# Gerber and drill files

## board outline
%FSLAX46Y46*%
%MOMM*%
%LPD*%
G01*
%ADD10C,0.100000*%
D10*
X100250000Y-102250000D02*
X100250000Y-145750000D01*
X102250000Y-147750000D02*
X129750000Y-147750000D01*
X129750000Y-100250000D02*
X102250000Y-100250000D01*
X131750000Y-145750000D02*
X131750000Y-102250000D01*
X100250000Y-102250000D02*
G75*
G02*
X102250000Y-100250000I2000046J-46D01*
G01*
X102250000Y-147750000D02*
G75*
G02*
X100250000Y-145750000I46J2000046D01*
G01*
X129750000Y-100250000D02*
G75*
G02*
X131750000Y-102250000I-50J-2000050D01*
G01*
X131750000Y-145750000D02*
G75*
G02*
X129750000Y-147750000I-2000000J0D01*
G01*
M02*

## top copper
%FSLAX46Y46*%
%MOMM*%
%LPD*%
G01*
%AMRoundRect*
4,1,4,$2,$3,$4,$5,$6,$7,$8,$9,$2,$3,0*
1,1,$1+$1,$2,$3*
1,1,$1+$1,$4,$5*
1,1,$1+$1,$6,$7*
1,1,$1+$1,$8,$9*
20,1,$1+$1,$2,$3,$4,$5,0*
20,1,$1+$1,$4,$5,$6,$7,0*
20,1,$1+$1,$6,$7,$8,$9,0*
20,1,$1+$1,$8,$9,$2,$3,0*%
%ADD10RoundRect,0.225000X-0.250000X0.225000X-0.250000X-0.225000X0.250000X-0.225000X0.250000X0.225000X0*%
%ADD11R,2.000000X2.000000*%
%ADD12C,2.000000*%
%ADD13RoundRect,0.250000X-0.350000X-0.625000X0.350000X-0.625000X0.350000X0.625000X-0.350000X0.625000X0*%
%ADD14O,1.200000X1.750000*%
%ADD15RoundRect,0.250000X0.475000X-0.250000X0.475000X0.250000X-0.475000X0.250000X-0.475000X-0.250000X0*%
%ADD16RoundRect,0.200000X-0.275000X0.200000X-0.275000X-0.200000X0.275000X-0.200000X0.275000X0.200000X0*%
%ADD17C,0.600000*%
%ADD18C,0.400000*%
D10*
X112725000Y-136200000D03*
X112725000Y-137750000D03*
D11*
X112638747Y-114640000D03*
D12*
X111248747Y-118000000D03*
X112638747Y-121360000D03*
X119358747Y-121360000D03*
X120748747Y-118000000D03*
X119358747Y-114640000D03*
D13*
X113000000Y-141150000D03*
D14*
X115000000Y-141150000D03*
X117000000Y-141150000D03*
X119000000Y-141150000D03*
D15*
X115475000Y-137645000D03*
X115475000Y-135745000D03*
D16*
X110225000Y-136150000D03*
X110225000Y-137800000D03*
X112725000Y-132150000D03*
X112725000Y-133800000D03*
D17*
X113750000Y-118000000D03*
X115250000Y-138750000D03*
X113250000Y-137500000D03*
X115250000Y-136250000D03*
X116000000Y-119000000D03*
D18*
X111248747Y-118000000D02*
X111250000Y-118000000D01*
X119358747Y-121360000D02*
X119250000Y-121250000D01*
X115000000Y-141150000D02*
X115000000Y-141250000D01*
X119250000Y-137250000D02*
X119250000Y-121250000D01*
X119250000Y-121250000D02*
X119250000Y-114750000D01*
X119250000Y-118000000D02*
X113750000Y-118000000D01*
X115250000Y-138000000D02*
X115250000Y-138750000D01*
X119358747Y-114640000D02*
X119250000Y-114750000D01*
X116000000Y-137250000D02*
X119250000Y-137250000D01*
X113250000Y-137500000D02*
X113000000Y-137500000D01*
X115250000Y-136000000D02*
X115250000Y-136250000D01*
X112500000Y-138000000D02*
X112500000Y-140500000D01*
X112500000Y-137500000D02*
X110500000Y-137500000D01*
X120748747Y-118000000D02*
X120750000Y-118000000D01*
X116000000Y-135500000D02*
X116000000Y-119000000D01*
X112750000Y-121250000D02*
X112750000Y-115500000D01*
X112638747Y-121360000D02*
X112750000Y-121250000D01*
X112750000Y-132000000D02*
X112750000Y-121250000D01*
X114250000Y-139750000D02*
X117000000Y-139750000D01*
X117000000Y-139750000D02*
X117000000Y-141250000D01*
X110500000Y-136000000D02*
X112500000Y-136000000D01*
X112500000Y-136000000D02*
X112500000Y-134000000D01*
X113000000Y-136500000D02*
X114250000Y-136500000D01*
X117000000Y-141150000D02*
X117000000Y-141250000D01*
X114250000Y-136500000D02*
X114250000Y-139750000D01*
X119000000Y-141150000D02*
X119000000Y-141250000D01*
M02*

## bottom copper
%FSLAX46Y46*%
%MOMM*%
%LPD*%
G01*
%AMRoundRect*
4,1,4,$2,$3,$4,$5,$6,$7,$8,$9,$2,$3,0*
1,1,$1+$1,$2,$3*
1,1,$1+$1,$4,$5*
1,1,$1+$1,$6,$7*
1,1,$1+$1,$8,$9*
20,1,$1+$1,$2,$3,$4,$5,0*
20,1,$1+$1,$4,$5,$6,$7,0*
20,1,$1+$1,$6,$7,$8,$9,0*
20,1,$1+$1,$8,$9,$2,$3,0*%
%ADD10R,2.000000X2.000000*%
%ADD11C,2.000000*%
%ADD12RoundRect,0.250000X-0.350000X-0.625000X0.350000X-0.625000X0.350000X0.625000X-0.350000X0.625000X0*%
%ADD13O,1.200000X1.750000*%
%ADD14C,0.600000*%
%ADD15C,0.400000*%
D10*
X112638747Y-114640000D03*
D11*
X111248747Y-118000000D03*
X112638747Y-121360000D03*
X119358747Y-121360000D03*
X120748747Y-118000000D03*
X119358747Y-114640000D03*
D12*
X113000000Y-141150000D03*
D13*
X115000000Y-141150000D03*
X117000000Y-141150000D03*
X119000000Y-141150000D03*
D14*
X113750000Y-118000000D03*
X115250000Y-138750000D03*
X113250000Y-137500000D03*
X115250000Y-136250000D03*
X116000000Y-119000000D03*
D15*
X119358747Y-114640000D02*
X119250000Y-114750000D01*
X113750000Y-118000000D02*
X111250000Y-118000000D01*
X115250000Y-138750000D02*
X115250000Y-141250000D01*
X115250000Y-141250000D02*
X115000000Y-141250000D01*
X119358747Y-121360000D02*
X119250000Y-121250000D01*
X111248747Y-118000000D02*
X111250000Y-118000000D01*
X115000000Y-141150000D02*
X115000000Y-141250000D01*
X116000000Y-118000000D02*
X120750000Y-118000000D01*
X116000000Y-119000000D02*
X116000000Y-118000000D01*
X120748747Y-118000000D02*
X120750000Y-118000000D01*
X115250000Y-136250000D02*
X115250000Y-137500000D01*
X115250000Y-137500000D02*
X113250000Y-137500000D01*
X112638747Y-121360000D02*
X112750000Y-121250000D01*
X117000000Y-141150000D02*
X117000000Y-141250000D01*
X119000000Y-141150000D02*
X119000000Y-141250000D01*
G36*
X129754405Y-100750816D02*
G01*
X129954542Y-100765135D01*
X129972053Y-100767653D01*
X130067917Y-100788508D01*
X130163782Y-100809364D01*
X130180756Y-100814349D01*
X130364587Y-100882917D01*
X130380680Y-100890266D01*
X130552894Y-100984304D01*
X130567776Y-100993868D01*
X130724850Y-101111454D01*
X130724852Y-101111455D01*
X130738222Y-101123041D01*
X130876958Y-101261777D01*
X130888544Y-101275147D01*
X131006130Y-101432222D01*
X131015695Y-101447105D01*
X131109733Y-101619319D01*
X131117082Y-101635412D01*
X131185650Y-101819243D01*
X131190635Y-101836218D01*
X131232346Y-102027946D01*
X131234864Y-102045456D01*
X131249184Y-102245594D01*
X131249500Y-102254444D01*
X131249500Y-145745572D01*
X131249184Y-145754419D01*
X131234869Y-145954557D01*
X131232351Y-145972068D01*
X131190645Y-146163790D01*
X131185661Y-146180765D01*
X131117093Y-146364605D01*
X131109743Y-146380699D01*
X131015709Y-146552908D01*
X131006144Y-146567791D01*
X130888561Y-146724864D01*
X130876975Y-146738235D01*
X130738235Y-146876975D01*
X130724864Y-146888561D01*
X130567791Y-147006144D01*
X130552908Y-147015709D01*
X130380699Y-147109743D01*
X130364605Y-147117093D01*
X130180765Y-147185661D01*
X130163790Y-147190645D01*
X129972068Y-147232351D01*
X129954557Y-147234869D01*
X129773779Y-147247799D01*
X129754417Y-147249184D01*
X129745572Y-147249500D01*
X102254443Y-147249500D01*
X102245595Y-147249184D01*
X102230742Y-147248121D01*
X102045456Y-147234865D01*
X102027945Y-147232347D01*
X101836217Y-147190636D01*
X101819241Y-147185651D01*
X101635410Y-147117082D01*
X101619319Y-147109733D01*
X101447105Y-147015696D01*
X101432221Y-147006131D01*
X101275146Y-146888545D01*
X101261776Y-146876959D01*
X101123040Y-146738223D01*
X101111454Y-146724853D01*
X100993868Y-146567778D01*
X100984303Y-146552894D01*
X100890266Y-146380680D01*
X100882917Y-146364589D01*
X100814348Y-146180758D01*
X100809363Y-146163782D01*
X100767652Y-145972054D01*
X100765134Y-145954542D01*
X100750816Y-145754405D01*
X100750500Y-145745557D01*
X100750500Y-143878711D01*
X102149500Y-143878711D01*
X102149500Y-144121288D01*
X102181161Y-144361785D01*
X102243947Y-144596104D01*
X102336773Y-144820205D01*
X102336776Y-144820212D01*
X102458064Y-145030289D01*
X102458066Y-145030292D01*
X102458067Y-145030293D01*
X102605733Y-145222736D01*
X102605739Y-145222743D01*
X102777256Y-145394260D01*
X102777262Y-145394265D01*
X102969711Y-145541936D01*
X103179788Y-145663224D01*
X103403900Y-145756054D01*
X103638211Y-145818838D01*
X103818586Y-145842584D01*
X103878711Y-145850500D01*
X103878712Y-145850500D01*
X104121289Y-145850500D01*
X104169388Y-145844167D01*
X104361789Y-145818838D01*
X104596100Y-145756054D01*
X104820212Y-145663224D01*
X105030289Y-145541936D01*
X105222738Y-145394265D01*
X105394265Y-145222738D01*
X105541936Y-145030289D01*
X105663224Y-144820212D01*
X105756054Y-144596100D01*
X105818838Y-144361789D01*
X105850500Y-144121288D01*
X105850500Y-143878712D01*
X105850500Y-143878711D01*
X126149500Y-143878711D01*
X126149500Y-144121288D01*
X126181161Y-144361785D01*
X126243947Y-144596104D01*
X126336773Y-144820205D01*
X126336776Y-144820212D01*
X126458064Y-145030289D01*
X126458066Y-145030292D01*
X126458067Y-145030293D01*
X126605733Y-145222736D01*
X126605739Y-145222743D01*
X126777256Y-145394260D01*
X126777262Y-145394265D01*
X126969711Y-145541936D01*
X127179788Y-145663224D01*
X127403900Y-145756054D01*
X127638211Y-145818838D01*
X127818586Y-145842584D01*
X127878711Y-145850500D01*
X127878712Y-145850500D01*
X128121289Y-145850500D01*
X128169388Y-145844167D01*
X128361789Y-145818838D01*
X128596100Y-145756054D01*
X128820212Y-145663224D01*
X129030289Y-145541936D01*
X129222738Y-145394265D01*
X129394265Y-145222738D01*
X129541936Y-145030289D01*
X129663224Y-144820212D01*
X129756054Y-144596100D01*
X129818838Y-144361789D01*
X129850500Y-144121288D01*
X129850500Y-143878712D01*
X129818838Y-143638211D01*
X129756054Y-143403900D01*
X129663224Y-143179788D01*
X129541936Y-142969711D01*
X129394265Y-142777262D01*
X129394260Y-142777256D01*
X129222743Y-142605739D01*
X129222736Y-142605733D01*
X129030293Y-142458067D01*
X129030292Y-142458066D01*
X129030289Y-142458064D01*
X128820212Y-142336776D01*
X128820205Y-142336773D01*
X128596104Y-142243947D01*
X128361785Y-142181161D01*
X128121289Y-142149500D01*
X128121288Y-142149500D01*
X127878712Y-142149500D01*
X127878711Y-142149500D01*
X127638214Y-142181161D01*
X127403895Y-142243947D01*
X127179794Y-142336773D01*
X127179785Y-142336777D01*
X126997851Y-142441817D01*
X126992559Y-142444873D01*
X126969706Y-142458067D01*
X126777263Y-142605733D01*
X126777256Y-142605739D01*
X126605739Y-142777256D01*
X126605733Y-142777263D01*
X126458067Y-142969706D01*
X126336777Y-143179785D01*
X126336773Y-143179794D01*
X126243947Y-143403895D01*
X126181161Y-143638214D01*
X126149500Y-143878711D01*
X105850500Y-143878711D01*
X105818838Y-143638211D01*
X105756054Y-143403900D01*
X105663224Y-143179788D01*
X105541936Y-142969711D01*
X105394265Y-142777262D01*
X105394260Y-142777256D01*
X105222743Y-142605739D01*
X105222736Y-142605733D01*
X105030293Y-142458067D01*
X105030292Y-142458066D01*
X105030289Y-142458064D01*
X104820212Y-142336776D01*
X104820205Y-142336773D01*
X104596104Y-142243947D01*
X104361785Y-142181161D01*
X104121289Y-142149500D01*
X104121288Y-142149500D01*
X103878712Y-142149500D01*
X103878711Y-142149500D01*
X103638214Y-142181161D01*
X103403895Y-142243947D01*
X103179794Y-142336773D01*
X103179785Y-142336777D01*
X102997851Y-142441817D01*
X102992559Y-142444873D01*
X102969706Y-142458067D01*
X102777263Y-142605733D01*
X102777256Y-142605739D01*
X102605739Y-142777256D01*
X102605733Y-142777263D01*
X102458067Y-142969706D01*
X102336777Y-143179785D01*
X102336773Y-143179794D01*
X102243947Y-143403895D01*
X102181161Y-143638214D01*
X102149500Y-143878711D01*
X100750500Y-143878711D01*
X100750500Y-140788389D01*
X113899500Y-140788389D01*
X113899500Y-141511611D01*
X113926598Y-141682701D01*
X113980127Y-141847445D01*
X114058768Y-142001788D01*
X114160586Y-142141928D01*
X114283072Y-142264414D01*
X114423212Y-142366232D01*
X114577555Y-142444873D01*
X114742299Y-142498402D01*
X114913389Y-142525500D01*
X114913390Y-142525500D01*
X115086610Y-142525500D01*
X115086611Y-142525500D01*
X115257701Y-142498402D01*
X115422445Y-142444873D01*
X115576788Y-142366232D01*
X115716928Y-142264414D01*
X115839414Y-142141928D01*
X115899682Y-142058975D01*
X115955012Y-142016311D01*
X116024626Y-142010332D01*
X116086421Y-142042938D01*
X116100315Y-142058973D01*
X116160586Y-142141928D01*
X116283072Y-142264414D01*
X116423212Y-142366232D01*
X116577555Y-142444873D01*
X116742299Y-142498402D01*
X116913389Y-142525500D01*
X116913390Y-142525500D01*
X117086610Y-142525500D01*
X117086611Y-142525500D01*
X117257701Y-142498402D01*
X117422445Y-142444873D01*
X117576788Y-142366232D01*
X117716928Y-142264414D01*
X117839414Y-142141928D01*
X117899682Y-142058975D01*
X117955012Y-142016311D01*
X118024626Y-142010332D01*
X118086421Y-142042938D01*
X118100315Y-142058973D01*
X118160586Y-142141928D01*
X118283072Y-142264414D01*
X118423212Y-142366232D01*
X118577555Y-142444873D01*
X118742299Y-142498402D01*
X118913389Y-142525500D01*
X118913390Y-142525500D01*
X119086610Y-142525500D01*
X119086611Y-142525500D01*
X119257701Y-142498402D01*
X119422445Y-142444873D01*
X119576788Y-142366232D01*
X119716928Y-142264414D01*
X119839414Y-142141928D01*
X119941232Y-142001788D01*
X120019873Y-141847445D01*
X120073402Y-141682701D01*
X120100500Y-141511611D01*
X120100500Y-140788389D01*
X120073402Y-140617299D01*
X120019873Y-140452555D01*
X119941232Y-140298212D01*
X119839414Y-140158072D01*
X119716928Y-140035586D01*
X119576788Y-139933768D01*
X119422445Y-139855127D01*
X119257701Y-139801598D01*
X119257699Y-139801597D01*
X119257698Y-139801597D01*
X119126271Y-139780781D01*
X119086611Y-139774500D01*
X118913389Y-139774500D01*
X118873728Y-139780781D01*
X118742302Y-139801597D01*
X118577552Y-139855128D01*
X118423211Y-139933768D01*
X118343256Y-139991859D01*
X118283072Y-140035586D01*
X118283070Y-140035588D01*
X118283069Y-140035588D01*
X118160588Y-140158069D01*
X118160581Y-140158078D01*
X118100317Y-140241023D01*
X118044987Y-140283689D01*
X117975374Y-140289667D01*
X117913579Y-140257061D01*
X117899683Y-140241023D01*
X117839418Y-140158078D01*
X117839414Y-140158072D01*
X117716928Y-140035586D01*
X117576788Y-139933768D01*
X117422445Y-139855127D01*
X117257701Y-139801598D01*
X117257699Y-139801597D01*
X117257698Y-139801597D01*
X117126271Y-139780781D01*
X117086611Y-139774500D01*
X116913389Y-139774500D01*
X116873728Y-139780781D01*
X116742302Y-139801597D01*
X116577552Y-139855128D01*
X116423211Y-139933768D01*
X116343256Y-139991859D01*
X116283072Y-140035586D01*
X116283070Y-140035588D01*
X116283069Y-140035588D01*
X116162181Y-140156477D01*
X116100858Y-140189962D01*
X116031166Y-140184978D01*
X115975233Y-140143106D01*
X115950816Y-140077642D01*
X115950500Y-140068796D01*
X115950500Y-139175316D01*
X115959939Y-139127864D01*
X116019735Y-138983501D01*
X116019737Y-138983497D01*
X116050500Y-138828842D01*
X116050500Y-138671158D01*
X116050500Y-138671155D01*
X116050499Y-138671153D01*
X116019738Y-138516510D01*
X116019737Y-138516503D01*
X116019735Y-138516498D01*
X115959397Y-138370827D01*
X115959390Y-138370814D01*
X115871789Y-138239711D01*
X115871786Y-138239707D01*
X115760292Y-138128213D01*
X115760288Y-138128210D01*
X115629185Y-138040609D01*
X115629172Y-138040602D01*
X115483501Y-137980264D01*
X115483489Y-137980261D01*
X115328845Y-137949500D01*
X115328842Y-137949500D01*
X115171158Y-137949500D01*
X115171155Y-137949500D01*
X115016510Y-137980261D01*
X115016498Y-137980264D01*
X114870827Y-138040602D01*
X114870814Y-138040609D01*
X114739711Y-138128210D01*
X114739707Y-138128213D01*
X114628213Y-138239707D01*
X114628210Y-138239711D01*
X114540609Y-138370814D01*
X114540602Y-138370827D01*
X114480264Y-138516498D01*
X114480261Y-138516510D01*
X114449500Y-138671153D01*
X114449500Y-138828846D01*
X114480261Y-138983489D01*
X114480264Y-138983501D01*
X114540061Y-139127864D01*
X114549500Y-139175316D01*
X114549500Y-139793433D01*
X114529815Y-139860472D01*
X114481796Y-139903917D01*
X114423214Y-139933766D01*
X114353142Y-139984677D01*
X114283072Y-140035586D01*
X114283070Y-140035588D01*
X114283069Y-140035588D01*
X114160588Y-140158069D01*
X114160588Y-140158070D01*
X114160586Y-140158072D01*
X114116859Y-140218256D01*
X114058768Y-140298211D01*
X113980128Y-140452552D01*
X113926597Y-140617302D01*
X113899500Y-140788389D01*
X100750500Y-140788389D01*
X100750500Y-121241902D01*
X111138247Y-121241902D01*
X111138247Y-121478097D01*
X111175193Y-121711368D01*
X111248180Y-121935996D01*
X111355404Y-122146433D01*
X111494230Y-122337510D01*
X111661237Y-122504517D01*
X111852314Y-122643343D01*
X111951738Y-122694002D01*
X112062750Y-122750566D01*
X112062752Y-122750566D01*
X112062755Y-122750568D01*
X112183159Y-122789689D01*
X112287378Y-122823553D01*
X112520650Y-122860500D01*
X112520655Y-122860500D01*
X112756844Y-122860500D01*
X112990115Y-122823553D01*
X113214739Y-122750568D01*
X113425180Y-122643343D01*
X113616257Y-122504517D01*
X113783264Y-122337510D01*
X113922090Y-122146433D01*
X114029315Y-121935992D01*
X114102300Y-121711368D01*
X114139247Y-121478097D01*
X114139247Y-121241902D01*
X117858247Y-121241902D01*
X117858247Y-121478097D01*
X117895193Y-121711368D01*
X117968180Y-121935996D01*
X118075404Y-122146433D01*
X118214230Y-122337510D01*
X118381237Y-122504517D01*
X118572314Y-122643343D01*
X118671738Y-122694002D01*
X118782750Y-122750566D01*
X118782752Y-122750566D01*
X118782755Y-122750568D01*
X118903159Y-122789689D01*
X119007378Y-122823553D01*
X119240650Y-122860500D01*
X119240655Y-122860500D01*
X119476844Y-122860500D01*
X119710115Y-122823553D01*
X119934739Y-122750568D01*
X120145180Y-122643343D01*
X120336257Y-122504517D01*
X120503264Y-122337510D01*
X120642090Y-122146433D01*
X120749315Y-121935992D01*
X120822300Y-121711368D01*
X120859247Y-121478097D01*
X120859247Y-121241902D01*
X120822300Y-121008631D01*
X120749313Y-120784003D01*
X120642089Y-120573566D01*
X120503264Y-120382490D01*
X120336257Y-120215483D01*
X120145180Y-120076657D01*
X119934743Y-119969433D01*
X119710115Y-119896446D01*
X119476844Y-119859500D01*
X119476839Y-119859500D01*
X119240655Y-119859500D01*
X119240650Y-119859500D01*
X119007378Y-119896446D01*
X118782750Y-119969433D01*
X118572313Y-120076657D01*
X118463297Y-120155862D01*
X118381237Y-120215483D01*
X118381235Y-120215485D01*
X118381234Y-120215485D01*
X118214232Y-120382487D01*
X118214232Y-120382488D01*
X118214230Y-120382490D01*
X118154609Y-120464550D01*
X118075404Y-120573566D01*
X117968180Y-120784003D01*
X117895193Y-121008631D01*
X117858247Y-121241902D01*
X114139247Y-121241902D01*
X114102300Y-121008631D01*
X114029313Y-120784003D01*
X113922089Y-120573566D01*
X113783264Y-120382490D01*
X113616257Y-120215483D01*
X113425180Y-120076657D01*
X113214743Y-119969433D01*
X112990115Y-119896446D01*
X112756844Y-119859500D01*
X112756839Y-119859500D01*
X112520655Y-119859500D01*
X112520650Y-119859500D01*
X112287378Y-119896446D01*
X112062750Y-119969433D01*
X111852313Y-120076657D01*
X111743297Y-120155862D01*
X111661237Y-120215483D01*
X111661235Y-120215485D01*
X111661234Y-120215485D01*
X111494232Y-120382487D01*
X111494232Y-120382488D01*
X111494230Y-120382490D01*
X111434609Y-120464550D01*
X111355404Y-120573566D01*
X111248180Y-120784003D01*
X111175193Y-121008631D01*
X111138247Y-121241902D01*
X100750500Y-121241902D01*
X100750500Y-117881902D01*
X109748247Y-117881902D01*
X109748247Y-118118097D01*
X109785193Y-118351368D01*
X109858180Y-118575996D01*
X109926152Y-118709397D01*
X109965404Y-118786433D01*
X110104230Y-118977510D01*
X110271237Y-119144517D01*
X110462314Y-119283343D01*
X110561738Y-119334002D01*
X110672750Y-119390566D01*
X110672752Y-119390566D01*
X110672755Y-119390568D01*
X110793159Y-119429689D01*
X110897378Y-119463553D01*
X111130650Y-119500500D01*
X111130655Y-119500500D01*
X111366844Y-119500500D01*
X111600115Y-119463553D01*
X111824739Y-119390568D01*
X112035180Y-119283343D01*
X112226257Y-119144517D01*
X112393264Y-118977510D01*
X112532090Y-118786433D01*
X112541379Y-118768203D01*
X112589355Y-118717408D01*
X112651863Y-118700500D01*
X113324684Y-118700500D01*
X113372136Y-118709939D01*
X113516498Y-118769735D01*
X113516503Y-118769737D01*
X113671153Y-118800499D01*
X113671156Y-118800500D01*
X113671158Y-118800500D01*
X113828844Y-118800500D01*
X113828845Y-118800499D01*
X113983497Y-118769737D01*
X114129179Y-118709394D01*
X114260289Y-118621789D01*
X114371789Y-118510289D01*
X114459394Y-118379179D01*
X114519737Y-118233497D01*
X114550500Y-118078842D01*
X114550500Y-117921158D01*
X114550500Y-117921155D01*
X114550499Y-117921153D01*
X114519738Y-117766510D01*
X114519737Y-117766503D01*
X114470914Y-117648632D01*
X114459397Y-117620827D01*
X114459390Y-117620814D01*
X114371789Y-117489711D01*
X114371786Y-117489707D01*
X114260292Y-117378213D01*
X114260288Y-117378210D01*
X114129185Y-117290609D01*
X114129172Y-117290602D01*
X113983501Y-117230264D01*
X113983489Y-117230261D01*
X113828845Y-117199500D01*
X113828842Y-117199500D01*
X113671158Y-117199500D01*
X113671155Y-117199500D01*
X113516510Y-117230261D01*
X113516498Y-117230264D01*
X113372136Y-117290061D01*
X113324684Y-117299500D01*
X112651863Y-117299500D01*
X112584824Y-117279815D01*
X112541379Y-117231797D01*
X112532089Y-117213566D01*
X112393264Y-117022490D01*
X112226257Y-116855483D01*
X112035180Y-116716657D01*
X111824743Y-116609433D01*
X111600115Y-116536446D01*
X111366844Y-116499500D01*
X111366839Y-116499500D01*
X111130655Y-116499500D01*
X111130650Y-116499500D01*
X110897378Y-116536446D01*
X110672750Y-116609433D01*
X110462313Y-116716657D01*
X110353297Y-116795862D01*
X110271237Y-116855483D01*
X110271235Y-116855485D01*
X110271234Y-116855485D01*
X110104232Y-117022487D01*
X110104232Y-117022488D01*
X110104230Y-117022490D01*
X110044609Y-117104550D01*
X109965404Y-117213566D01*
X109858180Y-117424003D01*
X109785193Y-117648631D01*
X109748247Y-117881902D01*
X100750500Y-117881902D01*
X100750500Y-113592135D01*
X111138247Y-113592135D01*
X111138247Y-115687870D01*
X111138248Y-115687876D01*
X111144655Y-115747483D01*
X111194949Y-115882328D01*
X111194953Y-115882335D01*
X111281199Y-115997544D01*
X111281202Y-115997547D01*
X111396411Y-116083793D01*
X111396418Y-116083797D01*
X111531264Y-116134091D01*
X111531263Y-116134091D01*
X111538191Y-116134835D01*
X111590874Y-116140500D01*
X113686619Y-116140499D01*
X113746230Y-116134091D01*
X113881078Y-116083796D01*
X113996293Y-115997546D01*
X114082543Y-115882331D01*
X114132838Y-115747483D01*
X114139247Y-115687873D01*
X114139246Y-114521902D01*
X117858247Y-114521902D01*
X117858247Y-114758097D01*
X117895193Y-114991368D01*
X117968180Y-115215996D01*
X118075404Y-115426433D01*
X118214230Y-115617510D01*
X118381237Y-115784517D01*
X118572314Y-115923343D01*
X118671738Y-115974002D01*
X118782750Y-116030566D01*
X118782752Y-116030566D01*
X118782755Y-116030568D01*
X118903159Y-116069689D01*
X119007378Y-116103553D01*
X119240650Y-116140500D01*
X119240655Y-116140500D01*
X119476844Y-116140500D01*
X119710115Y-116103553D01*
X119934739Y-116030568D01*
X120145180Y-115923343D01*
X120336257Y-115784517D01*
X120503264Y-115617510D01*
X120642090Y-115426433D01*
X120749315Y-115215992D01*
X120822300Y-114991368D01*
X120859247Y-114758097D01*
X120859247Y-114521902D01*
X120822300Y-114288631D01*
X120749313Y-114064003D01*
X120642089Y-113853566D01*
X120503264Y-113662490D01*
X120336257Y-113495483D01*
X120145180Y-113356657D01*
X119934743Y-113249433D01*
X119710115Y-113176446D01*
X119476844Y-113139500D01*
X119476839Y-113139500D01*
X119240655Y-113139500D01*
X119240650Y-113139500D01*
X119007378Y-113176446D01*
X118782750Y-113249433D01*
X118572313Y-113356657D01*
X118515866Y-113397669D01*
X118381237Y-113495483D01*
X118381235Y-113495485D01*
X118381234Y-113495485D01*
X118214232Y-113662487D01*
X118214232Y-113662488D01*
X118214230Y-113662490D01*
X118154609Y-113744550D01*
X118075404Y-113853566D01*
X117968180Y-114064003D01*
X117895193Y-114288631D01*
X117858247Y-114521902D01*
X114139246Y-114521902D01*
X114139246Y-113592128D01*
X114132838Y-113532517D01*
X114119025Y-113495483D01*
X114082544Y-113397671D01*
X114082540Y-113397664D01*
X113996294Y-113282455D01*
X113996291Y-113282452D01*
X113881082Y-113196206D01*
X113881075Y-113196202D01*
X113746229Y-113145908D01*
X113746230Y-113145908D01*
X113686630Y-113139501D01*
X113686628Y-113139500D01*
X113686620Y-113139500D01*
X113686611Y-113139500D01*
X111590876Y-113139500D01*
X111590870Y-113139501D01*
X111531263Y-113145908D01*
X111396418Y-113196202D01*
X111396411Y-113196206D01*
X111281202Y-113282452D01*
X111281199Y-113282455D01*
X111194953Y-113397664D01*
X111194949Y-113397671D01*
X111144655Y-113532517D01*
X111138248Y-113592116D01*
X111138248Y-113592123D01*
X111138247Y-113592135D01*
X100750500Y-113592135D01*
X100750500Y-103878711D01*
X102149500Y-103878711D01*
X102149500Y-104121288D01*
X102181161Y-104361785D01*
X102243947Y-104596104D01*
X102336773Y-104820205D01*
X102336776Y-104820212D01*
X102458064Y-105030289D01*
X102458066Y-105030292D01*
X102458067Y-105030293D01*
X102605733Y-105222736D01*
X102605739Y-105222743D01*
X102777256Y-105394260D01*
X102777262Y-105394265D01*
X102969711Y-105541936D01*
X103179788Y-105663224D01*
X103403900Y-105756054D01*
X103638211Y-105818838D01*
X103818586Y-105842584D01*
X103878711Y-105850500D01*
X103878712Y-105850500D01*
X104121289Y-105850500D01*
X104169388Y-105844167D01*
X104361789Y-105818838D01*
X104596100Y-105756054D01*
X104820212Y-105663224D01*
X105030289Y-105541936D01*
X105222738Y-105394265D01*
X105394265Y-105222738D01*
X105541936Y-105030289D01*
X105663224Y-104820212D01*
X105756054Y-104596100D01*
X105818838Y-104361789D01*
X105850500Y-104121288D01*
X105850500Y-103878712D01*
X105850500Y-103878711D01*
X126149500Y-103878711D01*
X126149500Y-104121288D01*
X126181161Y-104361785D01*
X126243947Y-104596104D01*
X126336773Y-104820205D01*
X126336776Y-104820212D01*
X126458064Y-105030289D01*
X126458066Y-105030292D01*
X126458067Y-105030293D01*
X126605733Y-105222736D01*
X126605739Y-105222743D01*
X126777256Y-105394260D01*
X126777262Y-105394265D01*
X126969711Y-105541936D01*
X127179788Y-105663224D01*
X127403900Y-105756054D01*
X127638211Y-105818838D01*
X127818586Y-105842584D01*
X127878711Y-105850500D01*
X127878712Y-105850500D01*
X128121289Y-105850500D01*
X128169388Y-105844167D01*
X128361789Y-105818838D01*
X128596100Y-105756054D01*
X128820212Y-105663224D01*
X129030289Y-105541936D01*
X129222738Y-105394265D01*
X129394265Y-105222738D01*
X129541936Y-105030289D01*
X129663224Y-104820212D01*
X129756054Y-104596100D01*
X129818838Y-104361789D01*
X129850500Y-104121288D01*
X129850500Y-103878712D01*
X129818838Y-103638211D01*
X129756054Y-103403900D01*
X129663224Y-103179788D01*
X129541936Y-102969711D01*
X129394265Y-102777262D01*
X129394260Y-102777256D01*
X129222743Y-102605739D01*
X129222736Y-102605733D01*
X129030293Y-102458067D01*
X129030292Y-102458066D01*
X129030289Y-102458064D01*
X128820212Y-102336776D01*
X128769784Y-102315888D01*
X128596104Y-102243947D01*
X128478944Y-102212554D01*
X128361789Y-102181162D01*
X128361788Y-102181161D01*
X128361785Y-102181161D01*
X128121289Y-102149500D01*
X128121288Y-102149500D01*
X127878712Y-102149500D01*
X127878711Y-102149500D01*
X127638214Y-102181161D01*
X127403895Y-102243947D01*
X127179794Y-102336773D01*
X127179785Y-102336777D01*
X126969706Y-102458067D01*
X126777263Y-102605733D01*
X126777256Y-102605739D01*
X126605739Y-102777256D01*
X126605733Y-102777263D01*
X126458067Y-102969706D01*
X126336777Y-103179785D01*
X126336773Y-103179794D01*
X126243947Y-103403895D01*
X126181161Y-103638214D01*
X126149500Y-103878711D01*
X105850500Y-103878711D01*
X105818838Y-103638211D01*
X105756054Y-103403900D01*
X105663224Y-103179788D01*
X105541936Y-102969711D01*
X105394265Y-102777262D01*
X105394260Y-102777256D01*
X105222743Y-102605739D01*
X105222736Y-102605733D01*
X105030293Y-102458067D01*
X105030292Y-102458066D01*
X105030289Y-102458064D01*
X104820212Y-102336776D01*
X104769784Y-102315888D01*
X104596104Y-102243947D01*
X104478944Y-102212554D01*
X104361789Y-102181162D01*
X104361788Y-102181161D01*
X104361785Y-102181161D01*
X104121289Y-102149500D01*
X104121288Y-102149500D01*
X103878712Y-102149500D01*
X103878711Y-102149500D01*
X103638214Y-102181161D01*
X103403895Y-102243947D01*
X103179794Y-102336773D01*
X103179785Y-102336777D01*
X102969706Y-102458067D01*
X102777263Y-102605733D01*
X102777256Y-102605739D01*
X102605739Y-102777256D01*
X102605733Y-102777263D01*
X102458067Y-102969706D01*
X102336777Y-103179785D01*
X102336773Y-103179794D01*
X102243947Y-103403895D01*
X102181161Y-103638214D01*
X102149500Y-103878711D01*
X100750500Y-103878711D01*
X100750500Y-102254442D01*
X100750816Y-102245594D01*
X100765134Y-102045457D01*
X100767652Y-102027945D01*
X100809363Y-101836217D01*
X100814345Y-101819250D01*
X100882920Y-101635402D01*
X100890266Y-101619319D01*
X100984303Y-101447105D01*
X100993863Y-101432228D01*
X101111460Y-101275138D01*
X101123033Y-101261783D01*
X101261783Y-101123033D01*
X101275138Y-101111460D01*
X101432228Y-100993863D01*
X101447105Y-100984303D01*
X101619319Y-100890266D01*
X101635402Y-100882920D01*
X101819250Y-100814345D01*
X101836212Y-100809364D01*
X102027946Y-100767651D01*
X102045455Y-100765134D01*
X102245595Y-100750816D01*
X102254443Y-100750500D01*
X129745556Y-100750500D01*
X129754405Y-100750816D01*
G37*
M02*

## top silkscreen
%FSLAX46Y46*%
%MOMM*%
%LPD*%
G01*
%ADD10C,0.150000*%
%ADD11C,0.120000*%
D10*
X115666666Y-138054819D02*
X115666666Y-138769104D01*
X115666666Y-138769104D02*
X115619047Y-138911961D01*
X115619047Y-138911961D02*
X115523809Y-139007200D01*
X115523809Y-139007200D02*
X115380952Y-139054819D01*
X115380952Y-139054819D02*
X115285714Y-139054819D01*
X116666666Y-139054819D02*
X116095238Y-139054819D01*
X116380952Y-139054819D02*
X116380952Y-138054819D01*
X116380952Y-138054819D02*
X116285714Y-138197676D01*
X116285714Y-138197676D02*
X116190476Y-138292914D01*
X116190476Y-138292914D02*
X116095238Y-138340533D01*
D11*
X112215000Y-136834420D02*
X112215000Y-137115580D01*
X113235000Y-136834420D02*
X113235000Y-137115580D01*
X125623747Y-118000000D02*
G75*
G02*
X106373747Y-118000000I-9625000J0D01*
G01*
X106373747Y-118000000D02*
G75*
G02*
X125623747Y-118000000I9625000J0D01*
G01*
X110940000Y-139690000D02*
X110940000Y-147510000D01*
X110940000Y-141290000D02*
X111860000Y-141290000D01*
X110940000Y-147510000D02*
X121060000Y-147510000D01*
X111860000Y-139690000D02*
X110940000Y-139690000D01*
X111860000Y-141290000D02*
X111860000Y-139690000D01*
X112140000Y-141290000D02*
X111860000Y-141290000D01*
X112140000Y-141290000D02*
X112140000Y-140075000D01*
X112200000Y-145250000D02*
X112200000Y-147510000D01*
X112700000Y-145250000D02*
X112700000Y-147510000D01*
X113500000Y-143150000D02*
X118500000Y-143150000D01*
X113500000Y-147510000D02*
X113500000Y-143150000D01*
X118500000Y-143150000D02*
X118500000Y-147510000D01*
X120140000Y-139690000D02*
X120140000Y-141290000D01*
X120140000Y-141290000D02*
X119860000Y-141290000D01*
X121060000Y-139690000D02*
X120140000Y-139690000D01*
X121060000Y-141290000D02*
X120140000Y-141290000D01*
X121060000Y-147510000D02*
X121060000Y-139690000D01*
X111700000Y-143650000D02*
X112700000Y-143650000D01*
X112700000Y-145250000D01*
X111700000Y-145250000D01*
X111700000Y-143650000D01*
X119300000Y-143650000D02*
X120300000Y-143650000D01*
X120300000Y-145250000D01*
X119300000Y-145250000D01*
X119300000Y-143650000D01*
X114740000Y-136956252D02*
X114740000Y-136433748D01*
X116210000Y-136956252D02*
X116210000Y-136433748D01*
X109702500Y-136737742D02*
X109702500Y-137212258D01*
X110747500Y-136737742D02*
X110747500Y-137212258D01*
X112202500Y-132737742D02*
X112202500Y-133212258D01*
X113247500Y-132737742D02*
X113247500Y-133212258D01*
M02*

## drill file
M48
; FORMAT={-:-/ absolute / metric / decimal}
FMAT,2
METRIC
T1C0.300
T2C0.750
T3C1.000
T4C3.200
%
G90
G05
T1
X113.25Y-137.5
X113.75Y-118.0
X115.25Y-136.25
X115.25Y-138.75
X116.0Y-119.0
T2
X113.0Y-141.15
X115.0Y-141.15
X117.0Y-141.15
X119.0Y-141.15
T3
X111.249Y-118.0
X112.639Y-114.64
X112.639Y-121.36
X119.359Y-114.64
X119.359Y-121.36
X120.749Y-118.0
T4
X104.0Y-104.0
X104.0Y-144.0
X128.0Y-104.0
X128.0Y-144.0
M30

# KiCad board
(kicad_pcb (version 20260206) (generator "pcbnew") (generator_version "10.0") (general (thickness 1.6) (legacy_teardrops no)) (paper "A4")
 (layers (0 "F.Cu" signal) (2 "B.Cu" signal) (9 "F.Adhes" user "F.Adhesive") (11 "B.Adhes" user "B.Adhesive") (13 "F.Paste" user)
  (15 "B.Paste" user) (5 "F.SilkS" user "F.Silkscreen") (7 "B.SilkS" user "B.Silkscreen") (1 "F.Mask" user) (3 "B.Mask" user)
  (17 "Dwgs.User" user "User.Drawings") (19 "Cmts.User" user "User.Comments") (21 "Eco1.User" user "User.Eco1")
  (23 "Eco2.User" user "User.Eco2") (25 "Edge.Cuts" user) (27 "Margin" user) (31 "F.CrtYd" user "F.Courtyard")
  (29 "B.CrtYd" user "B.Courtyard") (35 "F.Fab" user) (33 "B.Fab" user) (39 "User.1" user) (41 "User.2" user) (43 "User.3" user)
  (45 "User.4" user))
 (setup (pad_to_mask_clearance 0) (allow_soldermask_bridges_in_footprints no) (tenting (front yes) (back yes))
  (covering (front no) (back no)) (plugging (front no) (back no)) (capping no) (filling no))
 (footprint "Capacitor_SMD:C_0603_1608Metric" (layer "F.Cu") (at 112.725 136.975 -90)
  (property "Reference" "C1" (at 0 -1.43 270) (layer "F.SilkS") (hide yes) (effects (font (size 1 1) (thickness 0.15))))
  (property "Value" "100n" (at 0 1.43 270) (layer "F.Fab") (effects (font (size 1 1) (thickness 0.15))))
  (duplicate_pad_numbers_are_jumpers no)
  (fp_line (start -0.14058 0.51) (end 0.14058 0.51) (stroke (width 0.12) (type solid)) (layer "F.SilkS"))
  (fp_line (start -0.14058 -0.51) (end 0.14058 -0.51) (stroke (width 0.12) (type solid)) (layer "F.SilkS"))
  (pad "1" smd roundrect (at -0.775 0 270) (size 0.9 0.95) (layers "F.Cu" "F.Mask" "F.Paste") (roundrect_rratio 0.25) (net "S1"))
  (pad "2" smd roundrect (at 0.775 0 270) (size 0.9 0.95) (layers "F.Cu" "F.Mask" "F.Paste") (roundrect_rratio 0.25) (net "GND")))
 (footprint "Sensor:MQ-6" (layer "F.Cu") (at 112.638747 114.64)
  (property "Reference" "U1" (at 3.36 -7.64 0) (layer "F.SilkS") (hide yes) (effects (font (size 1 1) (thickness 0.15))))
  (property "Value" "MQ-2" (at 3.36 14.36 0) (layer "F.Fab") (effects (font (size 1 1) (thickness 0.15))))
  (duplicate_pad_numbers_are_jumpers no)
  (fp_circle (center 3.36 3.36) (end 12.985 3.36) (stroke (width 0.12) (type solid)) (fill no) (layer "F.SilkS"))
  (pad "1" thru_hole rect (at 0 0) (size 2 2) (drill 1) (layers "*.Cu" "*.Mask") (remove_unused_layers no) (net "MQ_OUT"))
  (pad "2" thru_hole circle (at -1.39 3.36) (size 2 2) (drill 1) (layers "*.Cu" "*.Mask") (remove_unused_layers no) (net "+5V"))
  (pad "3" thru_hole circle (at 0 6.72 90) (size 2 2) (drill 1) (layers "*.Cu" "*.Mask") (remove_unused_layers no) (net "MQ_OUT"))
  (pad "4" thru_hole circle (at 6.72 6.72 180) (size 2 2) (drill 1) (layers "*.Cu" "*.Mask") (remove_unused_layers no) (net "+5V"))
  (pad "5" thru_hole circle (at 8.11 3.36) (size 2 2) (drill 1) (layers "*.Cu" "*.Mask") (remove_unused_layers no) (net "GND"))
  (pad "6" thru_hole circle (at 6.72 0 270) (size 2 2) (drill 1) (layers "*.Cu" "*.Mask") (remove_unused_layers no) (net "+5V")))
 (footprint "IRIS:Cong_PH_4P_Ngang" (layer "F.Cu") (at 113 141.15)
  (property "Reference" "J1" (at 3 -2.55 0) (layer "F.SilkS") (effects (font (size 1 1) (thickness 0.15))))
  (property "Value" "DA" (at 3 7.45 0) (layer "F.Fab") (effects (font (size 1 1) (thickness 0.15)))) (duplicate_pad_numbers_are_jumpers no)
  (fp_line (start -2.06 -1.46) (end -2.06 6.36) (stroke (width 0.12) (type solid)) (layer "F.SilkS"))
  (fp_line (start -2.06 0.14) (end -1.14 0.14) (stroke (width 0.12) (type solid)) (layer "F.SilkS"))
  (fp_line (start -2.06 6.36) (end 8.06 6.36) (stroke (width 0.12) (type solid)) (layer "F.SilkS"))
  (fp_line (start -1.14 -1.46) (end -2.06 -1.46) (stroke (width 0.12) (type solid)) (layer "F.SilkS"))
  (fp_line (start -1.14 0.14) (end -1.14 -1.46) (stroke (width 0.12) (type solid)) (layer "F.SilkS"))
  (fp_line (start -0.86 0.14) (end -1.14 0.14) (stroke (width 0.12) (type solid)) (layer "F.SilkS"))
  (fp_line (start -0.86 0.14) (end -0.86 -1.075) (stroke (width 0.12) (type solid)) (layer "F.SilkS"))
  (fp_line (start -0.8 4.1) (end -0.8 6.36) (stroke (width 0.12) (type solid)) (layer "F.SilkS"))
  (fp_line (start -0.3 4.1) (end -0.3 6.36) (stroke (width 0.12) (type solid)) (layer "F.SilkS"))
  (fp_line (start 0.5 2) (end 5.5 2) (stroke (width 0.12) (type solid)) (layer "F.SilkS"))
  (fp_line (start 0.5 6.36) (end 0.5 2) (stroke (width 0.12) (type solid)) (layer "F.SilkS"))
  (fp_line (start 5.5 2) (end 5.5 6.36) (stroke (width 0.12) (type solid)) (layer "F.SilkS"))
  (fp_line (start 7.14 -1.46) (end 7.14 0.14) (stroke (width 0.12) (type solid)) (layer "F.SilkS"))
  (fp_line (start 7.14 0.14) (end 6.86 0.14) (stroke (width 0.12) (type solid)) (layer "F.SilkS"))
  (fp_line (start 8.06 -1.46) (end 7.14 -1.46) (stroke (width 0.12) (type solid)) (layer "F.SilkS"))
  (fp_line (start 8.06 0.14) (end 7.14 0.14) (stroke (width 0.12) (type solid)) (layer "F.SilkS"))
  (fp_line (start 8.06 6.36) (end 8.06 -1.46) (stroke (width 0.12) (type solid)) (layer "F.SilkS"))
  (fp_rect (start -1.3 2.5) (end -0.3 4.1) (stroke (width 0.12) (type solid)) (fill no) (layer "F.SilkS"))
  (fp_rect (start 6.3 2.5) (end 7.3 4.1) (stroke (width 0.12) (type solid)) (fill no) (layer "F.SilkS"))
  (pad "1" thru_hole roundrect (at 0 0) (size 1.2 1.75) (drill 0.75) (layers "*.Cu" "*.Mask") (remove_unused_layers no)
   (roundrect_rratio 0.208333) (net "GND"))
  (pad "2" thru_hole oval (at 2 0) (size 1.2 1.75) (drill 0.75) (layers "*.Cu" "*.Mask") (remove_unused_layers no) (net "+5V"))
  (pad "3" thru_hole oval (at 4 0) (size 1.2 1.75) (drill 0.75) (layers "*.Cu" "*.Mask") (remove_unused_layers no) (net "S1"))
  (pad "4" thru_hole oval (at 6 0) (size 1.2 1.75) (drill 0.75) (layers "*.Cu" "*.Mask") (remove_unused_layers no)
   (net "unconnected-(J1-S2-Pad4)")))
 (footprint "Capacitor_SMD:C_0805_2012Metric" (layer "F.Cu") (at 115.475 136.695 90)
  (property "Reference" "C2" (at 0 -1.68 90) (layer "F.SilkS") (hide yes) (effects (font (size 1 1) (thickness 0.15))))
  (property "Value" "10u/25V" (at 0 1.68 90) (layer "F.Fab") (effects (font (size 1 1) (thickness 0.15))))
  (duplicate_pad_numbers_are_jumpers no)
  (fp_line (start -0.261252 -0.735) (end 0.261252 -0.735) (stroke (width 0.12) (type solid)) (layer "F.SilkS"))
  (fp_line (start -0.261252 0.735) (end 0.261252 0.735) (stroke (width 0.12) (type solid)) (layer "F.SilkS"))
  (pad "1" smd roundrect (at -0.95 0 90) (size 1 1.45) (layers "F.Cu" "F.Mask" "F.Paste") (roundrect_rratio 0.25) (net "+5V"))
  (pad "2" smd roundrect (at 0.95 0 90) (size 1 1.45) (layers "F.Cu" "F.Mask" "F.Paste") (roundrect_rratio 0.25) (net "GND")))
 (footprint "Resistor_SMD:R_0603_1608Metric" (layer "F.Cu") (at 110.225 136.975 -90)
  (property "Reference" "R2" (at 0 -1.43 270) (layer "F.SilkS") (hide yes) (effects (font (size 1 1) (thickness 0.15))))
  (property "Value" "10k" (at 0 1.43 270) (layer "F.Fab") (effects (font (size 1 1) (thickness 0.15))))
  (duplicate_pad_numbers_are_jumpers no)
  (fp_line (start -0.237258 0.5225) (end 0.237258 0.5225) (stroke (width 0.12) (type solid)) (layer "F.SilkS"))
  (fp_line (start -0.237258 -0.5225) (end 0.237258 -0.5225) (stroke (width 0.12) (type solid)) (layer "F.SilkS"))
  (pad "1" smd roundrect (at -0.825 0 270) (size 0.8 0.95) (layers "F.Cu" "F.Mask" "F.Paste") (roundrect_rratio 0.25) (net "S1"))
  (pad "2" smd roundrect (at 0.825 0 270) (size 0.8 0.95) (layers "F.Cu" "F.Mask" "F.Paste") (roundrect_rratio 0.25) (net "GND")))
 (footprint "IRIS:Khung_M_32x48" (layer "F.Cu") (at 100 148)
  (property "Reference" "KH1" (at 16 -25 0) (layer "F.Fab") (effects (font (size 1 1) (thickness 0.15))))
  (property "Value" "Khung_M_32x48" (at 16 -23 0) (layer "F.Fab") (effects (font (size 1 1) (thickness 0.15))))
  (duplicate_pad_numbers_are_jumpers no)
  (fp_line (start 0.25 -45.75) (end 0.25 -2.25) (stroke (width 0.1) (type solid)) (layer "Edge.Cuts"))
  (fp_line (start 2.25 -0.25) (end 29.75 -0.25) (stroke (width 0.1) (type solid)) (layer "Edge.Cuts"))
  (fp_line (start 29.75 -47.75) (end 2.25 -47.75) (stroke (width 0.1) (type solid)) (layer "Edge.Cuts"))
  (fp_line (start 31.75 -2.25) (end 31.75 -45.75) (stroke (width 0.1) (type solid)) (layer "Edge.Cuts"))
  (fp_arc (start 0.25 -45.75) (mid 0.8358 -47.1642) (end 2.25 -47.75) (stroke (width 0.1) (type solid)) (layer "Edge.Cuts"))
  (fp_arc (start 2.25 -0.25) (mid 0.8358 -0.8358) (end 0.25 -2.25) (stroke (width 0.1) (type solid)) (layer "Edge.Cuts"))
  (fp_arc (start 29.75 -47.75) (mid 31.164199 -47.164199) (end 31.75 -45.75) (stroke (width 0.1) (type solid)) (layer "Edge.Cuts"))
  (fp_arc (start 31.75 -2.25) (mid 31.164214 -0.835786) (end 29.75 -0.25) (stroke (width 0.1) (type solid)) (layer "Edge.Cuts"))
  (pad "" np_thru_hole circle (at 4 -44) (size 3.2 3.2) (drill 3.2) (layers "*.Cu" "*.Mask"))
  (pad "" np_thru_hole circle (at 4 -4) (size 3.2 3.2) (drill 3.2) (layers "*.Cu" "*.Mask"))
  (pad "" np_thru_hole circle (at 28 -44) (size 3.2 3.2) (drill 3.2) (layers "*.Cu" "*.Mask"))
  (pad "" np_thru_hole circle (at 28 -4) (size 3.2 3.2) (drill 3.2) (layers "*.Cu" "*.Mask")))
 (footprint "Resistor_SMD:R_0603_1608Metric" (layer "F.Cu") (at 112.725 132.975 -90)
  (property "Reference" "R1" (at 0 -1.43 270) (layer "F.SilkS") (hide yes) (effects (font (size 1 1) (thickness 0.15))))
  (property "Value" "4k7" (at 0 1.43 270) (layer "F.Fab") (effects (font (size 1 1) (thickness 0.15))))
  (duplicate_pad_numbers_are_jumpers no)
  (fp_line (start -0.237258 0.5225) (end 0.237258 0.5225) (stroke (width 0.12) (type solid)) (layer "F.SilkS"))
  (fp_line (start -0.237258 -0.5225) (end 0.237258 -0.5225) (stroke (width 0.12) (type solid)) (layer "F.SilkS"))
  (pad "1" smd roundrect (at -0.825 0 270) (size 0.8 0.95) (layers "F.Cu" "F.Mask" "F.Paste") (roundrect_rratio 0.25) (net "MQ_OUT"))
  (pad "2" smd roundrect (at 0.825 0 270) (size 0.8 0.95) (layers "F.Cu" "F.Mask" "F.Paste") (roundrect_rratio 0.25) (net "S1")))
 (segment (start 111.248747 118) (end 111.25 118) (width 0.4) (layer "F.Cu") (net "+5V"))
 (segment (start 119.358747 121.36) (end 119.25 121.25) (width 0.4) (layer "F.Cu") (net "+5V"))
 (segment (start 115 141.15) (end 115 141.25) (width 0.4) (layer "F.Cu") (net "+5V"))
 (segment (start 119.25 137.25) (end 119.25 121.25) (width 0.4) (layer "F.Cu") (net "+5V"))
 (segment (start 119.25 121.25) (end 119.25 114.75) (width 0.4) (layer "F.Cu") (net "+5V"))
 (segment (start 119.25 118) (end 113.75 118) (width 0.4) (layer "F.Cu") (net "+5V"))
 (segment (start 115.25 138) (end 115.25 138.75) (width 0.4) (layer "F.Cu") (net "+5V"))
 (segment (start 119.358747 114.64) (end 119.25 114.75) (width 0.4) (layer "F.Cu") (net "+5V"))
 (segment (start 116 137.25) (end 119.25 137.25) (width 0.4) (layer "F.Cu") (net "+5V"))
 (via (at 113.75 118) (size 0.6) (drill 0.3) (layers "F.Cu" "B.Cu") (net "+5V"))
 (via (at 115.25 138.75) (size 0.6) (drill 0.3) (layers "F.Cu" "B.Cu") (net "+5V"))
 (segment (start 119.358747 114.64) (end 119.25 114.75) (width 0.4) (layer "B.Cu") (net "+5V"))
 (segment (start 113.75 118) (end 111.25 118) (width 0.4) (layer "B.Cu") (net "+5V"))
 (segment (start 115.25 138.75) (end 115.25 141.25) (width 0.4) (layer "B.Cu") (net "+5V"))
 (segment (start 115.25 141.25) (end 115 141.25) (width 0.4) (layer "B.Cu") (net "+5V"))
 (segment (start 119.358747 121.36) (end 119.25 121.25) (width 0.4) (layer "B.Cu") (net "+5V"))
 (segment (start 111.248747 118) (end 111.25 118) (width 0.4) (layer "B.Cu") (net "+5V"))
 (segment (start 115 141.15) (end 115 141.25) (width 0.4) (layer "B.Cu") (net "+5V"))
 (segment (start 113.25 137.5) (end 113 137.5) (width 0.4) (layer "F.Cu") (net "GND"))
 (segment (start 115.25 136) (end 115.25 136.25) (width 0.4) (layer "F.Cu") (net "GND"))
 (segment (start 112.5 138) (end 112.5 140.5) (width 0.4) (layer "F.Cu") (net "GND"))
 (segment (start 112.5 137.5) (end 110.5 137.5) (width 0.4) (layer "F.Cu") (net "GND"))
 (segment (start 120.748747 118) (end 120.75 118) (width 0.4) (layer "F.Cu") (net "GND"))
 (segment (start 116 135.5) (end 116 119) (width 0.4) (layer "F.Cu") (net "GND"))
 (via (at 113.25 137.5) (size 0.6) (drill 0.3) (layers "F.Cu" "B.Cu") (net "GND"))
 (via (at 115.25 136.25) (size 0.6) (drill 0.3) (layers "F.Cu" "B.Cu") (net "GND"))
 (via (at 116 119) (size 0.6) (drill 0.3) (layers "F.Cu" "B.Cu") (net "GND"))
 (segment (start 116 118) (end 120.75 118) (width 0.4) (layer "B.Cu") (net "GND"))
 (segment (start 116 119) (end 116 118) (width 0.4) (layer "B.Cu") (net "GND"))
 (segment (start 120.748747 118) (end 120.75 118) (width 0.4) (layer "B.Cu") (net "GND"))
 (segment (start 115.25 136.25) (end 115.25 137.5) (width 0.4) (layer "B.Cu") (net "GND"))
 (segment (start 115.25 137.5) (end 113.25 137.5) (width 0.4) (layer "B.Cu") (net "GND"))
 (segment (start 112.75 121.25) (end 112.75 115.5) (width 0.4) (layer "F.Cu") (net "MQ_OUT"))
 (segment (start 112.638747 121.36) (end 112.75 121.25) (width 0.4) (layer "F.Cu") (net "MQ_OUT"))
 (segment (start 112.75 132) (end 112.75 121.25) (width 0.4) (layer "F.Cu") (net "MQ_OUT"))
 (segment (start 112.638747 121.36) (end 112.75 121.25) (width 0.4) (layer "B.Cu") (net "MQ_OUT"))
 (segment (start 114.25 139.75) (end 117 139.75) (width 0.4) (layer "F.Cu") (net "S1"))
 (segment (start 117 139.75) (end 117 141.25) (width 0.4) (layer "F.Cu") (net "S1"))
 (segment (start 110.5 136) (end 112.5 136) (width 0.4) (layer "F.Cu") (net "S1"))
 (segment (start 112.5 136) (end 112.5 134) (width 0.4) (layer "F.Cu") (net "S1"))
 (segment (start 113 136.5) (end 114.25 136.5) (width 0.4) (layer "F.Cu") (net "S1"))
 (segment (start 117 141.15) (end 117 141.25) (width 0.4) (layer "F.Cu") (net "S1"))
 (segment (start 114.25 136.5) (end 114.25 139.75) (width 0.4) (layer "F.Cu") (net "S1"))
 (segment (start 117 141.15) (end 117 141.25) (width 0.4) (layer "B.Cu") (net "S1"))
 (segment (start 119 141.15) (end 119 141.25) (width 0.4) (layer "F.Cu") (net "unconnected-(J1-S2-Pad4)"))
 (segment (start 119 141.15) (end 119 141.25) (width 0.4) (layer "B.Cu") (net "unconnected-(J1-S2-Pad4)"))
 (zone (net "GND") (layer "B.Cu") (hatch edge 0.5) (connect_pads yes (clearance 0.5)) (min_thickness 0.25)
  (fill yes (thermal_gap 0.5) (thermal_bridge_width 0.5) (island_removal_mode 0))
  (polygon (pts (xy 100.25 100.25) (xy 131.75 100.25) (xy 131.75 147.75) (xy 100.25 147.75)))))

